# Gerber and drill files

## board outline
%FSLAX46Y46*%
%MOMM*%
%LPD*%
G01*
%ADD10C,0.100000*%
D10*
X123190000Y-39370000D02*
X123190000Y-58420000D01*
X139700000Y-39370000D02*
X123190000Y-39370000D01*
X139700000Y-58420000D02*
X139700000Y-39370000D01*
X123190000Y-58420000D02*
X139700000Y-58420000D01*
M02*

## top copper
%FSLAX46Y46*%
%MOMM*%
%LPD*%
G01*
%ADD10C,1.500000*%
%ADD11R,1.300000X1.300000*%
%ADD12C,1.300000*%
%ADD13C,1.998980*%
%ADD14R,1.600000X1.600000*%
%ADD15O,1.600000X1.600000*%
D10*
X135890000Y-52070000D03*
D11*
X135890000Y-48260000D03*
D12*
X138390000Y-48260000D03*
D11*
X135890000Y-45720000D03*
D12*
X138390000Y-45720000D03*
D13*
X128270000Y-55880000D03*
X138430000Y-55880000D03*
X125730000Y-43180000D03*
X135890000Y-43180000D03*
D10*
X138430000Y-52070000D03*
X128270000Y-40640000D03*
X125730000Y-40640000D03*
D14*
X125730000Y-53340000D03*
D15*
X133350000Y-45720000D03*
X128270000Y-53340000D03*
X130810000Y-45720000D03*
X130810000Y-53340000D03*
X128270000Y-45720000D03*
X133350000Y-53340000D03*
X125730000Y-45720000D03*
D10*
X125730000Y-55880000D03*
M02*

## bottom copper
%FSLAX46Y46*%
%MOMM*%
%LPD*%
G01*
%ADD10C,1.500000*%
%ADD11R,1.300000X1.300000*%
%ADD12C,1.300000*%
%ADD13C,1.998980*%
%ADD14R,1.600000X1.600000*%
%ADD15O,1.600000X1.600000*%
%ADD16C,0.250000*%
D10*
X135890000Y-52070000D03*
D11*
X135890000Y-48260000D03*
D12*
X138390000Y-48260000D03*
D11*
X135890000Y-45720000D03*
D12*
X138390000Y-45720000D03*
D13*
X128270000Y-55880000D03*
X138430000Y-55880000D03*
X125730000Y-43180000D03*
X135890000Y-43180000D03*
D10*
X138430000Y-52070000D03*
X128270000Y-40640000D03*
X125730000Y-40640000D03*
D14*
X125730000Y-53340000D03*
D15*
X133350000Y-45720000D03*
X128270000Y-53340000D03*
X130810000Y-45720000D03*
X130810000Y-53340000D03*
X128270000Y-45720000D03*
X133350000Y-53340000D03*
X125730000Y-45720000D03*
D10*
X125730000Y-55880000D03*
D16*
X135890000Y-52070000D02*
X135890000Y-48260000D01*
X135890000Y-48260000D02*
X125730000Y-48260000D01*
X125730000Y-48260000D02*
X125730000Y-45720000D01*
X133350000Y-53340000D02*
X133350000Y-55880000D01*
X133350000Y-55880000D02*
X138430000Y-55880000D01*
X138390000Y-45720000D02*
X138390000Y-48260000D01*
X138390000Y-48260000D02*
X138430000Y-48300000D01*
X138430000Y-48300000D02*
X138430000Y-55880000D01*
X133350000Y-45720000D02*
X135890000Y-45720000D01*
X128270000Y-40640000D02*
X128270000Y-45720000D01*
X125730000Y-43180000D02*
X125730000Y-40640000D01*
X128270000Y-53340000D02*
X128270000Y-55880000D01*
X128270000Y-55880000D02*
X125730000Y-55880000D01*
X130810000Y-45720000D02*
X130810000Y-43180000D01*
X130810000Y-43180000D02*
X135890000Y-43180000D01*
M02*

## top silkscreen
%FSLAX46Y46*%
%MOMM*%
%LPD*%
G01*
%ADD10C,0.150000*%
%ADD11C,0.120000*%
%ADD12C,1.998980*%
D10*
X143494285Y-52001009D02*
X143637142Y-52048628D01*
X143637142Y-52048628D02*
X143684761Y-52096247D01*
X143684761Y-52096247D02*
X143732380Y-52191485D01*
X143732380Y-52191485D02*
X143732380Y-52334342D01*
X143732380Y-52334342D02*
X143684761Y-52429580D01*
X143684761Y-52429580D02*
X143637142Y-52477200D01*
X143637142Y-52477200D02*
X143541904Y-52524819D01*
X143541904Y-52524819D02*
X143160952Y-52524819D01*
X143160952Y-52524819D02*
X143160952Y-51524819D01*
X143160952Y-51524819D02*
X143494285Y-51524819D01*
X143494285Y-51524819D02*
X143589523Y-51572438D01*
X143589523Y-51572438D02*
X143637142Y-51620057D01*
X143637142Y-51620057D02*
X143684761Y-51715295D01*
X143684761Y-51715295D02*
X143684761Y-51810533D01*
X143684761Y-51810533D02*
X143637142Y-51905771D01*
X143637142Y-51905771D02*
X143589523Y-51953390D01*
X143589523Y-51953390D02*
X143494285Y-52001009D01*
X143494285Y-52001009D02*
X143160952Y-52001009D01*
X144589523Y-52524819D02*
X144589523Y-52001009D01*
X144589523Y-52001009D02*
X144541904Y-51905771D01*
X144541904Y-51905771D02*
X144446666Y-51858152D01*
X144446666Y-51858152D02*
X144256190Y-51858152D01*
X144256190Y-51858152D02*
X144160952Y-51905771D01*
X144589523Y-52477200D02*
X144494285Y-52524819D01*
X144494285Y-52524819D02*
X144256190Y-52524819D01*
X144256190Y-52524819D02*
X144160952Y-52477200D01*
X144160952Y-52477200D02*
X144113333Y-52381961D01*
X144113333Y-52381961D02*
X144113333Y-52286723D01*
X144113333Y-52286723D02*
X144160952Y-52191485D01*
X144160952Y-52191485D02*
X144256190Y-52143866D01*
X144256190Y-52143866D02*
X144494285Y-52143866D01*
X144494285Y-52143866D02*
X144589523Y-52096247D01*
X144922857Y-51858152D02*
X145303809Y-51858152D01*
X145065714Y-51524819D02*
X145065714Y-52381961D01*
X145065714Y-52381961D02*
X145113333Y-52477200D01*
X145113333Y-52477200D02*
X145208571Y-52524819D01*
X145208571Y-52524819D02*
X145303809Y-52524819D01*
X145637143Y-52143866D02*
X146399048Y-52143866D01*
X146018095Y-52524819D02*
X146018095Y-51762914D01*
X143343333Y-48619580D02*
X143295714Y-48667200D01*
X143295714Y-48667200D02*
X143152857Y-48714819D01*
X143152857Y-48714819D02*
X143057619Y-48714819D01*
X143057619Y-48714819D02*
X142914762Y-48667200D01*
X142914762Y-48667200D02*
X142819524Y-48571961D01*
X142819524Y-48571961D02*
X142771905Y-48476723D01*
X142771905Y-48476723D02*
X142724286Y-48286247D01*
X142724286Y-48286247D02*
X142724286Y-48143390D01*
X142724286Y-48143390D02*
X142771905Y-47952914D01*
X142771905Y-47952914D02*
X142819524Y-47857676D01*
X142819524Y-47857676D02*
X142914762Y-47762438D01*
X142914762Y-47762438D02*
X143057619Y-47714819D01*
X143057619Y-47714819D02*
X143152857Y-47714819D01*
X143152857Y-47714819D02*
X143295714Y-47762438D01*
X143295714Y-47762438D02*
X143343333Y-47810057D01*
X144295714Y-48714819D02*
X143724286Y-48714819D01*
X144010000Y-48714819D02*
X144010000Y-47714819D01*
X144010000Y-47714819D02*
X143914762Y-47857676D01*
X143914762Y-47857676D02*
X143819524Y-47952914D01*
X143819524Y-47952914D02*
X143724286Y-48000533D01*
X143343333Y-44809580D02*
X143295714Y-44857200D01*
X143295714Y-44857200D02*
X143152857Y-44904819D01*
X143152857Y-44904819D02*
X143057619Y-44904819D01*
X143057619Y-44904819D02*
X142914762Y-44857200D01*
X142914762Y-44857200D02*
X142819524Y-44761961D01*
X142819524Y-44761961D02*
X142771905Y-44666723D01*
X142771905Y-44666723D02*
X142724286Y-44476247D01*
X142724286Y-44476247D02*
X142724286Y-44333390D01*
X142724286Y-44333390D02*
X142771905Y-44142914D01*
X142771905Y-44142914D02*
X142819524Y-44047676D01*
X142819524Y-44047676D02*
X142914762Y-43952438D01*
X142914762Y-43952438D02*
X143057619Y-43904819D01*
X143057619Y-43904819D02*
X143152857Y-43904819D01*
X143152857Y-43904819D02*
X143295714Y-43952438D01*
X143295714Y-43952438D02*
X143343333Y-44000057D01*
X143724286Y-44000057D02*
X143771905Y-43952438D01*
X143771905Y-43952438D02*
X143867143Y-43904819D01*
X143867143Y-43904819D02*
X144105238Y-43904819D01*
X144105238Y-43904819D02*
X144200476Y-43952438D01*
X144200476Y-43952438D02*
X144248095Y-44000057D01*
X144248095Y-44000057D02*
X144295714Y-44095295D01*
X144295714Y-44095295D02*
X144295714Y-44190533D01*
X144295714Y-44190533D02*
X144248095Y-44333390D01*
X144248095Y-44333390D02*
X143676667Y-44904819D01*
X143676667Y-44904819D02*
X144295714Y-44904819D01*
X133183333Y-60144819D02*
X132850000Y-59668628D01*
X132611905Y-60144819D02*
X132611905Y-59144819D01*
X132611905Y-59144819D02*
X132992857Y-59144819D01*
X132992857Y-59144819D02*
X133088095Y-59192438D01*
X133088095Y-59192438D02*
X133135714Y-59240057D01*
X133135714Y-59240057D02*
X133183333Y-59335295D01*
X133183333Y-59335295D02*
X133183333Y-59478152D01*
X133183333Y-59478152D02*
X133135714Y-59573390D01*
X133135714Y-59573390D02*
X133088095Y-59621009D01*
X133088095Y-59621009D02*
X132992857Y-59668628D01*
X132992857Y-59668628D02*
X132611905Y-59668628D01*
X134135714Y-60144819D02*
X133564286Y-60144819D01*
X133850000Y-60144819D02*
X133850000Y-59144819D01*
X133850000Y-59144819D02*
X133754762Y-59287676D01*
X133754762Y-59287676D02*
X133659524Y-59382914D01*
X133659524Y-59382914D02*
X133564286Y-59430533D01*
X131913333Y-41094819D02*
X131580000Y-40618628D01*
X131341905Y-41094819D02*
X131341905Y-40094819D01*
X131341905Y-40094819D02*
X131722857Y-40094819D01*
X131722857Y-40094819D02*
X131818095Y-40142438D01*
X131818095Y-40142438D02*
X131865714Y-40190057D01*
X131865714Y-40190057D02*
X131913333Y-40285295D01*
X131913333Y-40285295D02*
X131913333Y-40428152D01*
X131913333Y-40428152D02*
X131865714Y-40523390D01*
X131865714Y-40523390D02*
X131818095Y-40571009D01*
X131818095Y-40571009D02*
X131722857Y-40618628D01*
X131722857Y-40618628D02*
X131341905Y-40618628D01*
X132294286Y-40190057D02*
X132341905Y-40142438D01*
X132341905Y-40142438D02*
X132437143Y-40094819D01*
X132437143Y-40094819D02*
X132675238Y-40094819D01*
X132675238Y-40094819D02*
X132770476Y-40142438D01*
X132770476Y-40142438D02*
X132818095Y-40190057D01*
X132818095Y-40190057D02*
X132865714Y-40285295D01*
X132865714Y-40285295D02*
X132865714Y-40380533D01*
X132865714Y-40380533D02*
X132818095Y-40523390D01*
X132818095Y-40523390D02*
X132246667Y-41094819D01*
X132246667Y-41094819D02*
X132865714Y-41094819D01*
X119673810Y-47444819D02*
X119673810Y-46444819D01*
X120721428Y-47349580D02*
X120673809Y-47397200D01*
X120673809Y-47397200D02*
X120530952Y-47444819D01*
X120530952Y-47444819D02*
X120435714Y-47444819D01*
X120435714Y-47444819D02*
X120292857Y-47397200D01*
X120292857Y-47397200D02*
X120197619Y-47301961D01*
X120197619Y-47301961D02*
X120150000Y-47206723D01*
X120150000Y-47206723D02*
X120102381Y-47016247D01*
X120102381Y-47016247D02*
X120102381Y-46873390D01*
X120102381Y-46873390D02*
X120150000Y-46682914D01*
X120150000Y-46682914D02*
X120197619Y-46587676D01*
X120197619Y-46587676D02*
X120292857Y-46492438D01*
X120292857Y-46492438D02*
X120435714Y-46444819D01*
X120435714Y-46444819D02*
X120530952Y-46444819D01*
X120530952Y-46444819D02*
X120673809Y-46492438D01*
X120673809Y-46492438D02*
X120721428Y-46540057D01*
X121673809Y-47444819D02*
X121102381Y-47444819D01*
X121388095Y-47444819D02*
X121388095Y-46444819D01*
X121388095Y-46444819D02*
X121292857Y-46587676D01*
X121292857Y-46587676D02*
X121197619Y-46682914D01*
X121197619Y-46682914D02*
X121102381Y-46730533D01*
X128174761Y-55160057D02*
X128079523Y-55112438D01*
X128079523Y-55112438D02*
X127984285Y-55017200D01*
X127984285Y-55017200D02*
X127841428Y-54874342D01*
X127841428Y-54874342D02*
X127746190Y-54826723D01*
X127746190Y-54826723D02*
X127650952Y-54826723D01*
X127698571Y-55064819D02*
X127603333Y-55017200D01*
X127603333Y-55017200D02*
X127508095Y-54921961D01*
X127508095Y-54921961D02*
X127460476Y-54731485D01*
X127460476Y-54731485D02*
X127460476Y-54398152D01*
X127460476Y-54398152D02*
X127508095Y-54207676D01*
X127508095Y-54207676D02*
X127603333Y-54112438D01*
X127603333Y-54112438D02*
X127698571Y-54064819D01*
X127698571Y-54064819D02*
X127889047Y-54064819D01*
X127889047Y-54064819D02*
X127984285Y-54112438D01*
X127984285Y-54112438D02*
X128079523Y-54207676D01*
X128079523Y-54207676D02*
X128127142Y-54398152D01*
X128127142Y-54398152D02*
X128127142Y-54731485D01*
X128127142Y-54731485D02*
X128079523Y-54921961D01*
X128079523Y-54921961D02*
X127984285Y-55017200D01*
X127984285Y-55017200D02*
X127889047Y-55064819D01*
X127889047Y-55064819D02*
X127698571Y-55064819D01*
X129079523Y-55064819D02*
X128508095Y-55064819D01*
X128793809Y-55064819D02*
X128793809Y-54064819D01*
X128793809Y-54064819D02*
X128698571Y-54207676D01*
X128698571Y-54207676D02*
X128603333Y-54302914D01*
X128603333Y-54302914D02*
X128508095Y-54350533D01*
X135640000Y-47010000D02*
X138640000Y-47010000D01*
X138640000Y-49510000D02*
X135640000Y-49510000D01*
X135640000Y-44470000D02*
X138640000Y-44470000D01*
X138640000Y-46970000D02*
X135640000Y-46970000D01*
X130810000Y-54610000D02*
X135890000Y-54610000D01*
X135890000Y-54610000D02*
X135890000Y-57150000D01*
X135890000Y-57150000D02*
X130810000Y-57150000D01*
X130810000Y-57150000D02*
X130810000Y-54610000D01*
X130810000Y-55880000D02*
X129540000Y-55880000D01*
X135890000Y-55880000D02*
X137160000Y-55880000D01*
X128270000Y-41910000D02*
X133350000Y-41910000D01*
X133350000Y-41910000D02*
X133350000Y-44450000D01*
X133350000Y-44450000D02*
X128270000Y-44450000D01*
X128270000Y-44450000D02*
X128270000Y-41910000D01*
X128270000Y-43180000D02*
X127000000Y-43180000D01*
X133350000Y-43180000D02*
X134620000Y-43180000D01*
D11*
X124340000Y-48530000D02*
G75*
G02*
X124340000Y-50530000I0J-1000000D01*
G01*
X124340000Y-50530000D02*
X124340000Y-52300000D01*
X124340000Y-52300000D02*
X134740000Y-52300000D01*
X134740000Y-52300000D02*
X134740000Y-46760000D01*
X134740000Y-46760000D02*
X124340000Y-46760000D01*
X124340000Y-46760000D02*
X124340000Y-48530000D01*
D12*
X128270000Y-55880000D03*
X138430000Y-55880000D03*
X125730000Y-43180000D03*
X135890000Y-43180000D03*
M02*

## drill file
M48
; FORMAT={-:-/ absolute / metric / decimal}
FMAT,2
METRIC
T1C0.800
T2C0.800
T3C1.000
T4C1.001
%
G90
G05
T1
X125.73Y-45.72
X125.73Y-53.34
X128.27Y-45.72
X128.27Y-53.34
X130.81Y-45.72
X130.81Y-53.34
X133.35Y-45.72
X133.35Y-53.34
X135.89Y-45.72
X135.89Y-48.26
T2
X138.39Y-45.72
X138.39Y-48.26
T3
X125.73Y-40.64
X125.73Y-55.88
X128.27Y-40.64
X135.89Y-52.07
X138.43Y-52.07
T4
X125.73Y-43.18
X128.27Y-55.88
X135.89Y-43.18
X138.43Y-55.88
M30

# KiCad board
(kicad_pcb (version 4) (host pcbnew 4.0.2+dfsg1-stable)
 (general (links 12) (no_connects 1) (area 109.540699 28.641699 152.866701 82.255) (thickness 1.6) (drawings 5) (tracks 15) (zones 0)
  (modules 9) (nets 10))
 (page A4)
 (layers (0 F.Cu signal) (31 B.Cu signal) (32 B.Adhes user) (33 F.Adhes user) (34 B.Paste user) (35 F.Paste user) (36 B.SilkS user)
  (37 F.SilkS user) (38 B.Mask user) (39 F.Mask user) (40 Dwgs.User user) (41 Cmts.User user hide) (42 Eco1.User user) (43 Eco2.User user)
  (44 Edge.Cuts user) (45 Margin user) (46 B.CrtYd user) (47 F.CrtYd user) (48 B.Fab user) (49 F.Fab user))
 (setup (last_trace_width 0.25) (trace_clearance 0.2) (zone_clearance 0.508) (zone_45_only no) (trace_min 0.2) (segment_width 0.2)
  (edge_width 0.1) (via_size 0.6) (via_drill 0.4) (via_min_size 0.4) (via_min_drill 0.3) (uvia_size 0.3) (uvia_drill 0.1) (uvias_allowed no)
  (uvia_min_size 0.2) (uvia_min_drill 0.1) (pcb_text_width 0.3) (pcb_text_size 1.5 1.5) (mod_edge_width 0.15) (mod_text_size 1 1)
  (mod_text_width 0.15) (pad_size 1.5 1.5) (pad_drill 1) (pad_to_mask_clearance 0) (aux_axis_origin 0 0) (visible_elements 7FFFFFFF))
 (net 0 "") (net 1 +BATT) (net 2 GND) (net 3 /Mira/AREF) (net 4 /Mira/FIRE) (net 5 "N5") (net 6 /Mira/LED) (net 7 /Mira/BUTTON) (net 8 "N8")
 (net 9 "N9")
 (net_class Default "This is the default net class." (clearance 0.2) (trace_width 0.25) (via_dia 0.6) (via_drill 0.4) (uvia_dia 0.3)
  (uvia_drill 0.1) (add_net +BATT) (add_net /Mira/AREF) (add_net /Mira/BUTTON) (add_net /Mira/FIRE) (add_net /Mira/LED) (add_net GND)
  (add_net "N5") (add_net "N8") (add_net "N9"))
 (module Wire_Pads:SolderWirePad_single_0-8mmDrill (layer F.Cu) (at 133.35 73.66)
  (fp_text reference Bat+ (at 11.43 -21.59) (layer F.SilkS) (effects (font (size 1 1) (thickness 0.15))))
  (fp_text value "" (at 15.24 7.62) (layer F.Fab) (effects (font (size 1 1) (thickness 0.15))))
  (pad 1 thru_hole circle (at 2.54 -21.59) (size 1.5 1.5) (drill 1) (layers *.Cu *.Mask) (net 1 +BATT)))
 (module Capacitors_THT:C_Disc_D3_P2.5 (layer F.Cu) (at 135.89 48.26)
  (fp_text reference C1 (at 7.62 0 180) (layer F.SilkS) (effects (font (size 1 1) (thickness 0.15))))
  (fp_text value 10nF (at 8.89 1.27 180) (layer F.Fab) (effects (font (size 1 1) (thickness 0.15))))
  (fp_line (start -0.25 -1.25) (end 2.75 -1.25) (layer F.SilkS) (width 0.15))
  (fp_line (start 2.75 1.25) (end -0.25 1.25) (layer F.SilkS) (width 0.15))
  (pad 1 thru_hole rect (at 0 0) (size 1.3 1.3) (drill 0.8) (layers *.Cu *.Mask) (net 1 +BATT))
  (pad 2 thru_hole circle (at 2.5 0) (size 1.3 1.3) (drill 0.8001) (layers *.Cu *.Mask) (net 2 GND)))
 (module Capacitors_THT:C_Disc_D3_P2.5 (layer F.Cu) (at 135.89 45.72)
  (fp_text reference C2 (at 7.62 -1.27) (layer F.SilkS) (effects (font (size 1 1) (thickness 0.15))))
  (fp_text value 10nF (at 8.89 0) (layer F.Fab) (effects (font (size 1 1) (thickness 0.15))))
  (fp_line (start -0.25 -1.25) (end 2.75 -1.25) (layer F.SilkS) (width 0.15))
  (fp_line (start 2.75 1.25) (end -0.25 1.25) (layer F.SilkS) (width 0.15))
  (pad 1 thru_hole rect (at 0 0) (size 1.3 1.3) (drill 0.8) (layers *.Cu *.Mask) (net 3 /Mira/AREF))
  (pad 2 thru_hole circle (at 2.5 0) (size 1.3 1.3) (drill 0.8001) (layers *.Cu *.Mask) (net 2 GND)))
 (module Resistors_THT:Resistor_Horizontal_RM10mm (layer F.Cu) (at 128.27 55.88)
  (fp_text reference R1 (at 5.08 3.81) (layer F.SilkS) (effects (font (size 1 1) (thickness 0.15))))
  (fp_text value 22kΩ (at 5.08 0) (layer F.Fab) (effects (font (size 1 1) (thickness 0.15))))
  (fp_line (start 2.54 -1.27) (end 7.62 -1.27) (layer F.SilkS) (width 0.15))
  (fp_line (start 7.62 -1.27) (end 7.62 1.27) (layer F.SilkS) (width 0.15))
  (fp_line (start 7.62 1.27) (end 2.54 1.27) (layer F.SilkS) (width 0.15))
  (fp_line (start 2.54 1.27) (end 2.54 -1.27) (layer F.SilkS) (width 0.15))
  (fp_line (start 2.54 0) (end 1.27 0) (layer F.SilkS) (width 0.15))
  (fp_line (start 7.62 0) (end 8.89 0) (layer F.SilkS) (width 0.15))
  (pad 1 thru_hole circle (at 0 0) (size 1.99898 1.99898) (drill 1.00076) (layers *.Cu *.SilkS *.Mask) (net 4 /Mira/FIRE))
  (pad 2 thru_hole circle (at 10.16 0) (size 1.99898 1.99898) (drill 1.00076) (layers *.Cu *.SilkS *.Mask) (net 2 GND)))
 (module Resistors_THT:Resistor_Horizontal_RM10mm (layer F.Cu) (at 125.73 43.18)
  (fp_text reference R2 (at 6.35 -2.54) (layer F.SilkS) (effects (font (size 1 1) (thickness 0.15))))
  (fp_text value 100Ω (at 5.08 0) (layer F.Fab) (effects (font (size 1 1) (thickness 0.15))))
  (fp_line (start 2.54 -1.27) (end 7.62 -1.27) (layer F.SilkS) (width 0.15))
  (fp_line (start 7.62 -1.27) (end 7.62 1.27) (layer F.SilkS) (width 0.15))
  (fp_line (start 7.62 1.27) (end 2.54 1.27) (layer F.SilkS) (width 0.15))
  (fp_line (start 2.54 1.27) (end 2.54 -1.27) (layer F.SilkS) (width 0.15))
  (fp_line (start 2.54 0) (end 1.27 0) (layer F.SilkS) (width 0.15))
  (fp_line (start 7.62 0) (end 8.89 0) (layer F.SilkS) (width 0.15))
  (pad 1 thru_hole circle (at 0 0) (size 1.99898 1.99898) (drill 1.00076) (layers *.Cu *.SilkS *.Mask) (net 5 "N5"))
  (pad 2 thru_hole circle (at 10.16 0) (size 1.99898 1.99898) (drill 1.00076) (layers *.Cu *.SilkS *.Mask) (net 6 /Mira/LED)))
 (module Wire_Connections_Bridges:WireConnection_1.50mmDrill (layer F.Cu) (at 138.43 34.29)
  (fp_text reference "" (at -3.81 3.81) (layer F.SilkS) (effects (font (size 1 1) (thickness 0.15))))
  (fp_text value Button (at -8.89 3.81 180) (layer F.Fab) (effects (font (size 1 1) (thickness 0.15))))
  (pad 1 thru_hole circle (at 0 17.78) (size 1.5 1.5) (drill 1) (layers *.Cu *.Mask) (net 2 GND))
  (pad 2 thru_hole circle (at -10.16 6.35) (size 1.5 1.5) (drill 1) (layers *.Cu *.Mask) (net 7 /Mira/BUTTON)))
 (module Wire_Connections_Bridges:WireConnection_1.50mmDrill (layer F.Cu) (at 124.46 57.15)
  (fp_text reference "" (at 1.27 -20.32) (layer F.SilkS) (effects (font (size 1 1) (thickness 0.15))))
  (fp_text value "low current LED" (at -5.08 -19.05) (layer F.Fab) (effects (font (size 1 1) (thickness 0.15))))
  (pad 2 thru_hole circle (at 1.27 -16.51) (size 1.5 1.5) (drill 1) (layers *.Cu *.Mask) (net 5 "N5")))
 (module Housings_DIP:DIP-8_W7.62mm (layer F.Cu) (at 125.73 53.34 90)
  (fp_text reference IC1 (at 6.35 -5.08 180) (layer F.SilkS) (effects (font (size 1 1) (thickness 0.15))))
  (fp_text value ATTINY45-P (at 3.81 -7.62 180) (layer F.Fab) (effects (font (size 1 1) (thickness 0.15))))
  (fp_arc (start 3.81 -1.39) (end 2.81 -1.39) (angle -180) (layer F.SilkS) (width 0.12))
  (fp_line (start 2.81 -1.39) (end 1.04 -1.39) (layer F.SilkS) (width 0.12))
  (fp_line (start 1.04 -1.39) (end 1.04 9.01) (layer F.SilkS) (width 0.12))
  (fp_line (start 1.04 9.01) (end 6.58 9.01) (layer F.SilkS) (width 0.12))
  (fp_line (start 6.58 9.01) (end 6.58 -1.39) (layer F.SilkS) (width 0.12))
  (fp_line (start 6.58 -1.39) (end 4.81 -1.39) (layer F.SilkS) (width 0.12))
  (pad 1 thru_hole rect (at 0 0 90) (size 1.6 1.6) (drill 0.8) (layers *.Cu *.Mask) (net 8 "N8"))
  (pad 5 thru_hole oval (at 7.62 7.62 90) (size 1.6 1.6) (drill 0.8) (layers *.Cu *.Mask) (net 3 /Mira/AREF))
  (pad 2 thru_hole oval (at 0 2.54 90) (size 1.6 1.6) (drill 0.8) (layers *.Cu *.Mask) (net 4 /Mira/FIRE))
  (pad 6 thru_hole oval (at 7.62 5.08 90) (size 1.6 1.6) (drill 0.8) (layers *.Cu *.Mask) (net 6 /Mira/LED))
  (pad 3 thru_hole oval (at 0 5.08 90) (size 1.6 1.6) (drill 0.8) (layers *.Cu *.Mask) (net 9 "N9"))
  (pad 7 thru_hole oval (at 7.62 2.54 90) (size 1.6 1.6) (drill 0.8) (layers *.Cu *.Mask) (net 7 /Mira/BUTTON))
  (pad 4 thru_hole oval (at 0 7.62 90) (size 1.6 1.6) (drill 0.8) (layers *.Cu *.Mask) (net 2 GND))
  (pad 8 thru_hole oval (at 7.62 0 90) (size 1.6 1.6) (drill 0.8) (layers *.Cu *.Mask) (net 1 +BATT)))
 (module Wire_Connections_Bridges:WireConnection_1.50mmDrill (layer F.Cu) (at 113.03 60.96)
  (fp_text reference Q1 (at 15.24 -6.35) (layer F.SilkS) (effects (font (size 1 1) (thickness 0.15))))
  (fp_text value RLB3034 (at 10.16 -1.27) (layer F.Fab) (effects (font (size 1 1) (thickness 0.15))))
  (pad 2 thru_hole circle (at 12.7 -5.08) (size 1.5 1.5) (drill 1) (layers *.Cu *.Mask) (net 4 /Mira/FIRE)))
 (gr_line (start 123.19 39.37) (end 123.19 58.42) (angle 90) (layer Edge.Cuts) (width 0.1))
 (gr_line (start 139.7 39.37) (end 123.19 39.37) (angle 90) (layer Edge.Cuts) (width 0.1))
 (gr_line (start 139.7 58.42) (end 139.7 39.37) (angle 90) (layer Edge.Cuts) (width 0.1))
 (gr_line (start 123.19 58.42) (end 139.7 58.42) (angle 90) (layer Edge.Cuts) (width 0.1))
 (segment (start 135.89 52.07) (end 135.89 48.26) (width 0.25) (layer B.Cu) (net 1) (status C00000))
 (segment (start 135.89 48.26) (end 125.73 48.26) (width 0.25) (layer B.Cu) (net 1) (status 400000))
 (segment (start 125.73 48.26) (end 125.73 45.72) (width 0.25) (layer B.Cu) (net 1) (status 800000))
 (segment (start 133.35 53.34) (end 133.35 55.88) (width 0.25) (layer B.Cu) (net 2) (status 400000))
 (segment (start 133.35 55.88) (end 138.43 55.88) (width 0.25) (layer B.Cu) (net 2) (status 800000))
 (segment (start 138.39 45.72) (end 138.39 48.26) (width 0.25) (layer B.Cu) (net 2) (status C00000))
 (segment (start 138.39 48.26) (end 138.43 48.3) (width 0.25) (layer B.Cu) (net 2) (status C00000))
 (segment (start 138.43 48.3) (end 138.43 55.88) (width 0.25) (layer B.Cu) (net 2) (status C00000))
 (segment (start 133.35 45.72) (end 135.89 45.72) (width 0.25) (layer B.Cu) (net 3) (status C00000))
 (segment (start 128.27 40.64) (end 128.27 45.72) (width 0.25) (layer B.Cu) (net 7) (status C00000))
 (segment (start 125.73 43.18) (end 125.73 40.64) (width 0.25) (layer B.Cu) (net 5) (status C00000))
 (segment (start 128.27 53.34) (end 128.27 55.88) (width 0.25) (layer B.Cu) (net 4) (status C00000))
 (segment (start 128.27 55.88) (end 125.73 55.88) (width 0.25) (layer B.Cu) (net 4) (status C00000))
 (segment (start 130.81 45.72) (end 130.81 43.18) (width 0.25) (layer B.Cu) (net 6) (status 400000))
 (segment (start 130.81 43.18) (end 135.89 43.18) (width 0.25) (layer B.Cu) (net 6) (status 800000)))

